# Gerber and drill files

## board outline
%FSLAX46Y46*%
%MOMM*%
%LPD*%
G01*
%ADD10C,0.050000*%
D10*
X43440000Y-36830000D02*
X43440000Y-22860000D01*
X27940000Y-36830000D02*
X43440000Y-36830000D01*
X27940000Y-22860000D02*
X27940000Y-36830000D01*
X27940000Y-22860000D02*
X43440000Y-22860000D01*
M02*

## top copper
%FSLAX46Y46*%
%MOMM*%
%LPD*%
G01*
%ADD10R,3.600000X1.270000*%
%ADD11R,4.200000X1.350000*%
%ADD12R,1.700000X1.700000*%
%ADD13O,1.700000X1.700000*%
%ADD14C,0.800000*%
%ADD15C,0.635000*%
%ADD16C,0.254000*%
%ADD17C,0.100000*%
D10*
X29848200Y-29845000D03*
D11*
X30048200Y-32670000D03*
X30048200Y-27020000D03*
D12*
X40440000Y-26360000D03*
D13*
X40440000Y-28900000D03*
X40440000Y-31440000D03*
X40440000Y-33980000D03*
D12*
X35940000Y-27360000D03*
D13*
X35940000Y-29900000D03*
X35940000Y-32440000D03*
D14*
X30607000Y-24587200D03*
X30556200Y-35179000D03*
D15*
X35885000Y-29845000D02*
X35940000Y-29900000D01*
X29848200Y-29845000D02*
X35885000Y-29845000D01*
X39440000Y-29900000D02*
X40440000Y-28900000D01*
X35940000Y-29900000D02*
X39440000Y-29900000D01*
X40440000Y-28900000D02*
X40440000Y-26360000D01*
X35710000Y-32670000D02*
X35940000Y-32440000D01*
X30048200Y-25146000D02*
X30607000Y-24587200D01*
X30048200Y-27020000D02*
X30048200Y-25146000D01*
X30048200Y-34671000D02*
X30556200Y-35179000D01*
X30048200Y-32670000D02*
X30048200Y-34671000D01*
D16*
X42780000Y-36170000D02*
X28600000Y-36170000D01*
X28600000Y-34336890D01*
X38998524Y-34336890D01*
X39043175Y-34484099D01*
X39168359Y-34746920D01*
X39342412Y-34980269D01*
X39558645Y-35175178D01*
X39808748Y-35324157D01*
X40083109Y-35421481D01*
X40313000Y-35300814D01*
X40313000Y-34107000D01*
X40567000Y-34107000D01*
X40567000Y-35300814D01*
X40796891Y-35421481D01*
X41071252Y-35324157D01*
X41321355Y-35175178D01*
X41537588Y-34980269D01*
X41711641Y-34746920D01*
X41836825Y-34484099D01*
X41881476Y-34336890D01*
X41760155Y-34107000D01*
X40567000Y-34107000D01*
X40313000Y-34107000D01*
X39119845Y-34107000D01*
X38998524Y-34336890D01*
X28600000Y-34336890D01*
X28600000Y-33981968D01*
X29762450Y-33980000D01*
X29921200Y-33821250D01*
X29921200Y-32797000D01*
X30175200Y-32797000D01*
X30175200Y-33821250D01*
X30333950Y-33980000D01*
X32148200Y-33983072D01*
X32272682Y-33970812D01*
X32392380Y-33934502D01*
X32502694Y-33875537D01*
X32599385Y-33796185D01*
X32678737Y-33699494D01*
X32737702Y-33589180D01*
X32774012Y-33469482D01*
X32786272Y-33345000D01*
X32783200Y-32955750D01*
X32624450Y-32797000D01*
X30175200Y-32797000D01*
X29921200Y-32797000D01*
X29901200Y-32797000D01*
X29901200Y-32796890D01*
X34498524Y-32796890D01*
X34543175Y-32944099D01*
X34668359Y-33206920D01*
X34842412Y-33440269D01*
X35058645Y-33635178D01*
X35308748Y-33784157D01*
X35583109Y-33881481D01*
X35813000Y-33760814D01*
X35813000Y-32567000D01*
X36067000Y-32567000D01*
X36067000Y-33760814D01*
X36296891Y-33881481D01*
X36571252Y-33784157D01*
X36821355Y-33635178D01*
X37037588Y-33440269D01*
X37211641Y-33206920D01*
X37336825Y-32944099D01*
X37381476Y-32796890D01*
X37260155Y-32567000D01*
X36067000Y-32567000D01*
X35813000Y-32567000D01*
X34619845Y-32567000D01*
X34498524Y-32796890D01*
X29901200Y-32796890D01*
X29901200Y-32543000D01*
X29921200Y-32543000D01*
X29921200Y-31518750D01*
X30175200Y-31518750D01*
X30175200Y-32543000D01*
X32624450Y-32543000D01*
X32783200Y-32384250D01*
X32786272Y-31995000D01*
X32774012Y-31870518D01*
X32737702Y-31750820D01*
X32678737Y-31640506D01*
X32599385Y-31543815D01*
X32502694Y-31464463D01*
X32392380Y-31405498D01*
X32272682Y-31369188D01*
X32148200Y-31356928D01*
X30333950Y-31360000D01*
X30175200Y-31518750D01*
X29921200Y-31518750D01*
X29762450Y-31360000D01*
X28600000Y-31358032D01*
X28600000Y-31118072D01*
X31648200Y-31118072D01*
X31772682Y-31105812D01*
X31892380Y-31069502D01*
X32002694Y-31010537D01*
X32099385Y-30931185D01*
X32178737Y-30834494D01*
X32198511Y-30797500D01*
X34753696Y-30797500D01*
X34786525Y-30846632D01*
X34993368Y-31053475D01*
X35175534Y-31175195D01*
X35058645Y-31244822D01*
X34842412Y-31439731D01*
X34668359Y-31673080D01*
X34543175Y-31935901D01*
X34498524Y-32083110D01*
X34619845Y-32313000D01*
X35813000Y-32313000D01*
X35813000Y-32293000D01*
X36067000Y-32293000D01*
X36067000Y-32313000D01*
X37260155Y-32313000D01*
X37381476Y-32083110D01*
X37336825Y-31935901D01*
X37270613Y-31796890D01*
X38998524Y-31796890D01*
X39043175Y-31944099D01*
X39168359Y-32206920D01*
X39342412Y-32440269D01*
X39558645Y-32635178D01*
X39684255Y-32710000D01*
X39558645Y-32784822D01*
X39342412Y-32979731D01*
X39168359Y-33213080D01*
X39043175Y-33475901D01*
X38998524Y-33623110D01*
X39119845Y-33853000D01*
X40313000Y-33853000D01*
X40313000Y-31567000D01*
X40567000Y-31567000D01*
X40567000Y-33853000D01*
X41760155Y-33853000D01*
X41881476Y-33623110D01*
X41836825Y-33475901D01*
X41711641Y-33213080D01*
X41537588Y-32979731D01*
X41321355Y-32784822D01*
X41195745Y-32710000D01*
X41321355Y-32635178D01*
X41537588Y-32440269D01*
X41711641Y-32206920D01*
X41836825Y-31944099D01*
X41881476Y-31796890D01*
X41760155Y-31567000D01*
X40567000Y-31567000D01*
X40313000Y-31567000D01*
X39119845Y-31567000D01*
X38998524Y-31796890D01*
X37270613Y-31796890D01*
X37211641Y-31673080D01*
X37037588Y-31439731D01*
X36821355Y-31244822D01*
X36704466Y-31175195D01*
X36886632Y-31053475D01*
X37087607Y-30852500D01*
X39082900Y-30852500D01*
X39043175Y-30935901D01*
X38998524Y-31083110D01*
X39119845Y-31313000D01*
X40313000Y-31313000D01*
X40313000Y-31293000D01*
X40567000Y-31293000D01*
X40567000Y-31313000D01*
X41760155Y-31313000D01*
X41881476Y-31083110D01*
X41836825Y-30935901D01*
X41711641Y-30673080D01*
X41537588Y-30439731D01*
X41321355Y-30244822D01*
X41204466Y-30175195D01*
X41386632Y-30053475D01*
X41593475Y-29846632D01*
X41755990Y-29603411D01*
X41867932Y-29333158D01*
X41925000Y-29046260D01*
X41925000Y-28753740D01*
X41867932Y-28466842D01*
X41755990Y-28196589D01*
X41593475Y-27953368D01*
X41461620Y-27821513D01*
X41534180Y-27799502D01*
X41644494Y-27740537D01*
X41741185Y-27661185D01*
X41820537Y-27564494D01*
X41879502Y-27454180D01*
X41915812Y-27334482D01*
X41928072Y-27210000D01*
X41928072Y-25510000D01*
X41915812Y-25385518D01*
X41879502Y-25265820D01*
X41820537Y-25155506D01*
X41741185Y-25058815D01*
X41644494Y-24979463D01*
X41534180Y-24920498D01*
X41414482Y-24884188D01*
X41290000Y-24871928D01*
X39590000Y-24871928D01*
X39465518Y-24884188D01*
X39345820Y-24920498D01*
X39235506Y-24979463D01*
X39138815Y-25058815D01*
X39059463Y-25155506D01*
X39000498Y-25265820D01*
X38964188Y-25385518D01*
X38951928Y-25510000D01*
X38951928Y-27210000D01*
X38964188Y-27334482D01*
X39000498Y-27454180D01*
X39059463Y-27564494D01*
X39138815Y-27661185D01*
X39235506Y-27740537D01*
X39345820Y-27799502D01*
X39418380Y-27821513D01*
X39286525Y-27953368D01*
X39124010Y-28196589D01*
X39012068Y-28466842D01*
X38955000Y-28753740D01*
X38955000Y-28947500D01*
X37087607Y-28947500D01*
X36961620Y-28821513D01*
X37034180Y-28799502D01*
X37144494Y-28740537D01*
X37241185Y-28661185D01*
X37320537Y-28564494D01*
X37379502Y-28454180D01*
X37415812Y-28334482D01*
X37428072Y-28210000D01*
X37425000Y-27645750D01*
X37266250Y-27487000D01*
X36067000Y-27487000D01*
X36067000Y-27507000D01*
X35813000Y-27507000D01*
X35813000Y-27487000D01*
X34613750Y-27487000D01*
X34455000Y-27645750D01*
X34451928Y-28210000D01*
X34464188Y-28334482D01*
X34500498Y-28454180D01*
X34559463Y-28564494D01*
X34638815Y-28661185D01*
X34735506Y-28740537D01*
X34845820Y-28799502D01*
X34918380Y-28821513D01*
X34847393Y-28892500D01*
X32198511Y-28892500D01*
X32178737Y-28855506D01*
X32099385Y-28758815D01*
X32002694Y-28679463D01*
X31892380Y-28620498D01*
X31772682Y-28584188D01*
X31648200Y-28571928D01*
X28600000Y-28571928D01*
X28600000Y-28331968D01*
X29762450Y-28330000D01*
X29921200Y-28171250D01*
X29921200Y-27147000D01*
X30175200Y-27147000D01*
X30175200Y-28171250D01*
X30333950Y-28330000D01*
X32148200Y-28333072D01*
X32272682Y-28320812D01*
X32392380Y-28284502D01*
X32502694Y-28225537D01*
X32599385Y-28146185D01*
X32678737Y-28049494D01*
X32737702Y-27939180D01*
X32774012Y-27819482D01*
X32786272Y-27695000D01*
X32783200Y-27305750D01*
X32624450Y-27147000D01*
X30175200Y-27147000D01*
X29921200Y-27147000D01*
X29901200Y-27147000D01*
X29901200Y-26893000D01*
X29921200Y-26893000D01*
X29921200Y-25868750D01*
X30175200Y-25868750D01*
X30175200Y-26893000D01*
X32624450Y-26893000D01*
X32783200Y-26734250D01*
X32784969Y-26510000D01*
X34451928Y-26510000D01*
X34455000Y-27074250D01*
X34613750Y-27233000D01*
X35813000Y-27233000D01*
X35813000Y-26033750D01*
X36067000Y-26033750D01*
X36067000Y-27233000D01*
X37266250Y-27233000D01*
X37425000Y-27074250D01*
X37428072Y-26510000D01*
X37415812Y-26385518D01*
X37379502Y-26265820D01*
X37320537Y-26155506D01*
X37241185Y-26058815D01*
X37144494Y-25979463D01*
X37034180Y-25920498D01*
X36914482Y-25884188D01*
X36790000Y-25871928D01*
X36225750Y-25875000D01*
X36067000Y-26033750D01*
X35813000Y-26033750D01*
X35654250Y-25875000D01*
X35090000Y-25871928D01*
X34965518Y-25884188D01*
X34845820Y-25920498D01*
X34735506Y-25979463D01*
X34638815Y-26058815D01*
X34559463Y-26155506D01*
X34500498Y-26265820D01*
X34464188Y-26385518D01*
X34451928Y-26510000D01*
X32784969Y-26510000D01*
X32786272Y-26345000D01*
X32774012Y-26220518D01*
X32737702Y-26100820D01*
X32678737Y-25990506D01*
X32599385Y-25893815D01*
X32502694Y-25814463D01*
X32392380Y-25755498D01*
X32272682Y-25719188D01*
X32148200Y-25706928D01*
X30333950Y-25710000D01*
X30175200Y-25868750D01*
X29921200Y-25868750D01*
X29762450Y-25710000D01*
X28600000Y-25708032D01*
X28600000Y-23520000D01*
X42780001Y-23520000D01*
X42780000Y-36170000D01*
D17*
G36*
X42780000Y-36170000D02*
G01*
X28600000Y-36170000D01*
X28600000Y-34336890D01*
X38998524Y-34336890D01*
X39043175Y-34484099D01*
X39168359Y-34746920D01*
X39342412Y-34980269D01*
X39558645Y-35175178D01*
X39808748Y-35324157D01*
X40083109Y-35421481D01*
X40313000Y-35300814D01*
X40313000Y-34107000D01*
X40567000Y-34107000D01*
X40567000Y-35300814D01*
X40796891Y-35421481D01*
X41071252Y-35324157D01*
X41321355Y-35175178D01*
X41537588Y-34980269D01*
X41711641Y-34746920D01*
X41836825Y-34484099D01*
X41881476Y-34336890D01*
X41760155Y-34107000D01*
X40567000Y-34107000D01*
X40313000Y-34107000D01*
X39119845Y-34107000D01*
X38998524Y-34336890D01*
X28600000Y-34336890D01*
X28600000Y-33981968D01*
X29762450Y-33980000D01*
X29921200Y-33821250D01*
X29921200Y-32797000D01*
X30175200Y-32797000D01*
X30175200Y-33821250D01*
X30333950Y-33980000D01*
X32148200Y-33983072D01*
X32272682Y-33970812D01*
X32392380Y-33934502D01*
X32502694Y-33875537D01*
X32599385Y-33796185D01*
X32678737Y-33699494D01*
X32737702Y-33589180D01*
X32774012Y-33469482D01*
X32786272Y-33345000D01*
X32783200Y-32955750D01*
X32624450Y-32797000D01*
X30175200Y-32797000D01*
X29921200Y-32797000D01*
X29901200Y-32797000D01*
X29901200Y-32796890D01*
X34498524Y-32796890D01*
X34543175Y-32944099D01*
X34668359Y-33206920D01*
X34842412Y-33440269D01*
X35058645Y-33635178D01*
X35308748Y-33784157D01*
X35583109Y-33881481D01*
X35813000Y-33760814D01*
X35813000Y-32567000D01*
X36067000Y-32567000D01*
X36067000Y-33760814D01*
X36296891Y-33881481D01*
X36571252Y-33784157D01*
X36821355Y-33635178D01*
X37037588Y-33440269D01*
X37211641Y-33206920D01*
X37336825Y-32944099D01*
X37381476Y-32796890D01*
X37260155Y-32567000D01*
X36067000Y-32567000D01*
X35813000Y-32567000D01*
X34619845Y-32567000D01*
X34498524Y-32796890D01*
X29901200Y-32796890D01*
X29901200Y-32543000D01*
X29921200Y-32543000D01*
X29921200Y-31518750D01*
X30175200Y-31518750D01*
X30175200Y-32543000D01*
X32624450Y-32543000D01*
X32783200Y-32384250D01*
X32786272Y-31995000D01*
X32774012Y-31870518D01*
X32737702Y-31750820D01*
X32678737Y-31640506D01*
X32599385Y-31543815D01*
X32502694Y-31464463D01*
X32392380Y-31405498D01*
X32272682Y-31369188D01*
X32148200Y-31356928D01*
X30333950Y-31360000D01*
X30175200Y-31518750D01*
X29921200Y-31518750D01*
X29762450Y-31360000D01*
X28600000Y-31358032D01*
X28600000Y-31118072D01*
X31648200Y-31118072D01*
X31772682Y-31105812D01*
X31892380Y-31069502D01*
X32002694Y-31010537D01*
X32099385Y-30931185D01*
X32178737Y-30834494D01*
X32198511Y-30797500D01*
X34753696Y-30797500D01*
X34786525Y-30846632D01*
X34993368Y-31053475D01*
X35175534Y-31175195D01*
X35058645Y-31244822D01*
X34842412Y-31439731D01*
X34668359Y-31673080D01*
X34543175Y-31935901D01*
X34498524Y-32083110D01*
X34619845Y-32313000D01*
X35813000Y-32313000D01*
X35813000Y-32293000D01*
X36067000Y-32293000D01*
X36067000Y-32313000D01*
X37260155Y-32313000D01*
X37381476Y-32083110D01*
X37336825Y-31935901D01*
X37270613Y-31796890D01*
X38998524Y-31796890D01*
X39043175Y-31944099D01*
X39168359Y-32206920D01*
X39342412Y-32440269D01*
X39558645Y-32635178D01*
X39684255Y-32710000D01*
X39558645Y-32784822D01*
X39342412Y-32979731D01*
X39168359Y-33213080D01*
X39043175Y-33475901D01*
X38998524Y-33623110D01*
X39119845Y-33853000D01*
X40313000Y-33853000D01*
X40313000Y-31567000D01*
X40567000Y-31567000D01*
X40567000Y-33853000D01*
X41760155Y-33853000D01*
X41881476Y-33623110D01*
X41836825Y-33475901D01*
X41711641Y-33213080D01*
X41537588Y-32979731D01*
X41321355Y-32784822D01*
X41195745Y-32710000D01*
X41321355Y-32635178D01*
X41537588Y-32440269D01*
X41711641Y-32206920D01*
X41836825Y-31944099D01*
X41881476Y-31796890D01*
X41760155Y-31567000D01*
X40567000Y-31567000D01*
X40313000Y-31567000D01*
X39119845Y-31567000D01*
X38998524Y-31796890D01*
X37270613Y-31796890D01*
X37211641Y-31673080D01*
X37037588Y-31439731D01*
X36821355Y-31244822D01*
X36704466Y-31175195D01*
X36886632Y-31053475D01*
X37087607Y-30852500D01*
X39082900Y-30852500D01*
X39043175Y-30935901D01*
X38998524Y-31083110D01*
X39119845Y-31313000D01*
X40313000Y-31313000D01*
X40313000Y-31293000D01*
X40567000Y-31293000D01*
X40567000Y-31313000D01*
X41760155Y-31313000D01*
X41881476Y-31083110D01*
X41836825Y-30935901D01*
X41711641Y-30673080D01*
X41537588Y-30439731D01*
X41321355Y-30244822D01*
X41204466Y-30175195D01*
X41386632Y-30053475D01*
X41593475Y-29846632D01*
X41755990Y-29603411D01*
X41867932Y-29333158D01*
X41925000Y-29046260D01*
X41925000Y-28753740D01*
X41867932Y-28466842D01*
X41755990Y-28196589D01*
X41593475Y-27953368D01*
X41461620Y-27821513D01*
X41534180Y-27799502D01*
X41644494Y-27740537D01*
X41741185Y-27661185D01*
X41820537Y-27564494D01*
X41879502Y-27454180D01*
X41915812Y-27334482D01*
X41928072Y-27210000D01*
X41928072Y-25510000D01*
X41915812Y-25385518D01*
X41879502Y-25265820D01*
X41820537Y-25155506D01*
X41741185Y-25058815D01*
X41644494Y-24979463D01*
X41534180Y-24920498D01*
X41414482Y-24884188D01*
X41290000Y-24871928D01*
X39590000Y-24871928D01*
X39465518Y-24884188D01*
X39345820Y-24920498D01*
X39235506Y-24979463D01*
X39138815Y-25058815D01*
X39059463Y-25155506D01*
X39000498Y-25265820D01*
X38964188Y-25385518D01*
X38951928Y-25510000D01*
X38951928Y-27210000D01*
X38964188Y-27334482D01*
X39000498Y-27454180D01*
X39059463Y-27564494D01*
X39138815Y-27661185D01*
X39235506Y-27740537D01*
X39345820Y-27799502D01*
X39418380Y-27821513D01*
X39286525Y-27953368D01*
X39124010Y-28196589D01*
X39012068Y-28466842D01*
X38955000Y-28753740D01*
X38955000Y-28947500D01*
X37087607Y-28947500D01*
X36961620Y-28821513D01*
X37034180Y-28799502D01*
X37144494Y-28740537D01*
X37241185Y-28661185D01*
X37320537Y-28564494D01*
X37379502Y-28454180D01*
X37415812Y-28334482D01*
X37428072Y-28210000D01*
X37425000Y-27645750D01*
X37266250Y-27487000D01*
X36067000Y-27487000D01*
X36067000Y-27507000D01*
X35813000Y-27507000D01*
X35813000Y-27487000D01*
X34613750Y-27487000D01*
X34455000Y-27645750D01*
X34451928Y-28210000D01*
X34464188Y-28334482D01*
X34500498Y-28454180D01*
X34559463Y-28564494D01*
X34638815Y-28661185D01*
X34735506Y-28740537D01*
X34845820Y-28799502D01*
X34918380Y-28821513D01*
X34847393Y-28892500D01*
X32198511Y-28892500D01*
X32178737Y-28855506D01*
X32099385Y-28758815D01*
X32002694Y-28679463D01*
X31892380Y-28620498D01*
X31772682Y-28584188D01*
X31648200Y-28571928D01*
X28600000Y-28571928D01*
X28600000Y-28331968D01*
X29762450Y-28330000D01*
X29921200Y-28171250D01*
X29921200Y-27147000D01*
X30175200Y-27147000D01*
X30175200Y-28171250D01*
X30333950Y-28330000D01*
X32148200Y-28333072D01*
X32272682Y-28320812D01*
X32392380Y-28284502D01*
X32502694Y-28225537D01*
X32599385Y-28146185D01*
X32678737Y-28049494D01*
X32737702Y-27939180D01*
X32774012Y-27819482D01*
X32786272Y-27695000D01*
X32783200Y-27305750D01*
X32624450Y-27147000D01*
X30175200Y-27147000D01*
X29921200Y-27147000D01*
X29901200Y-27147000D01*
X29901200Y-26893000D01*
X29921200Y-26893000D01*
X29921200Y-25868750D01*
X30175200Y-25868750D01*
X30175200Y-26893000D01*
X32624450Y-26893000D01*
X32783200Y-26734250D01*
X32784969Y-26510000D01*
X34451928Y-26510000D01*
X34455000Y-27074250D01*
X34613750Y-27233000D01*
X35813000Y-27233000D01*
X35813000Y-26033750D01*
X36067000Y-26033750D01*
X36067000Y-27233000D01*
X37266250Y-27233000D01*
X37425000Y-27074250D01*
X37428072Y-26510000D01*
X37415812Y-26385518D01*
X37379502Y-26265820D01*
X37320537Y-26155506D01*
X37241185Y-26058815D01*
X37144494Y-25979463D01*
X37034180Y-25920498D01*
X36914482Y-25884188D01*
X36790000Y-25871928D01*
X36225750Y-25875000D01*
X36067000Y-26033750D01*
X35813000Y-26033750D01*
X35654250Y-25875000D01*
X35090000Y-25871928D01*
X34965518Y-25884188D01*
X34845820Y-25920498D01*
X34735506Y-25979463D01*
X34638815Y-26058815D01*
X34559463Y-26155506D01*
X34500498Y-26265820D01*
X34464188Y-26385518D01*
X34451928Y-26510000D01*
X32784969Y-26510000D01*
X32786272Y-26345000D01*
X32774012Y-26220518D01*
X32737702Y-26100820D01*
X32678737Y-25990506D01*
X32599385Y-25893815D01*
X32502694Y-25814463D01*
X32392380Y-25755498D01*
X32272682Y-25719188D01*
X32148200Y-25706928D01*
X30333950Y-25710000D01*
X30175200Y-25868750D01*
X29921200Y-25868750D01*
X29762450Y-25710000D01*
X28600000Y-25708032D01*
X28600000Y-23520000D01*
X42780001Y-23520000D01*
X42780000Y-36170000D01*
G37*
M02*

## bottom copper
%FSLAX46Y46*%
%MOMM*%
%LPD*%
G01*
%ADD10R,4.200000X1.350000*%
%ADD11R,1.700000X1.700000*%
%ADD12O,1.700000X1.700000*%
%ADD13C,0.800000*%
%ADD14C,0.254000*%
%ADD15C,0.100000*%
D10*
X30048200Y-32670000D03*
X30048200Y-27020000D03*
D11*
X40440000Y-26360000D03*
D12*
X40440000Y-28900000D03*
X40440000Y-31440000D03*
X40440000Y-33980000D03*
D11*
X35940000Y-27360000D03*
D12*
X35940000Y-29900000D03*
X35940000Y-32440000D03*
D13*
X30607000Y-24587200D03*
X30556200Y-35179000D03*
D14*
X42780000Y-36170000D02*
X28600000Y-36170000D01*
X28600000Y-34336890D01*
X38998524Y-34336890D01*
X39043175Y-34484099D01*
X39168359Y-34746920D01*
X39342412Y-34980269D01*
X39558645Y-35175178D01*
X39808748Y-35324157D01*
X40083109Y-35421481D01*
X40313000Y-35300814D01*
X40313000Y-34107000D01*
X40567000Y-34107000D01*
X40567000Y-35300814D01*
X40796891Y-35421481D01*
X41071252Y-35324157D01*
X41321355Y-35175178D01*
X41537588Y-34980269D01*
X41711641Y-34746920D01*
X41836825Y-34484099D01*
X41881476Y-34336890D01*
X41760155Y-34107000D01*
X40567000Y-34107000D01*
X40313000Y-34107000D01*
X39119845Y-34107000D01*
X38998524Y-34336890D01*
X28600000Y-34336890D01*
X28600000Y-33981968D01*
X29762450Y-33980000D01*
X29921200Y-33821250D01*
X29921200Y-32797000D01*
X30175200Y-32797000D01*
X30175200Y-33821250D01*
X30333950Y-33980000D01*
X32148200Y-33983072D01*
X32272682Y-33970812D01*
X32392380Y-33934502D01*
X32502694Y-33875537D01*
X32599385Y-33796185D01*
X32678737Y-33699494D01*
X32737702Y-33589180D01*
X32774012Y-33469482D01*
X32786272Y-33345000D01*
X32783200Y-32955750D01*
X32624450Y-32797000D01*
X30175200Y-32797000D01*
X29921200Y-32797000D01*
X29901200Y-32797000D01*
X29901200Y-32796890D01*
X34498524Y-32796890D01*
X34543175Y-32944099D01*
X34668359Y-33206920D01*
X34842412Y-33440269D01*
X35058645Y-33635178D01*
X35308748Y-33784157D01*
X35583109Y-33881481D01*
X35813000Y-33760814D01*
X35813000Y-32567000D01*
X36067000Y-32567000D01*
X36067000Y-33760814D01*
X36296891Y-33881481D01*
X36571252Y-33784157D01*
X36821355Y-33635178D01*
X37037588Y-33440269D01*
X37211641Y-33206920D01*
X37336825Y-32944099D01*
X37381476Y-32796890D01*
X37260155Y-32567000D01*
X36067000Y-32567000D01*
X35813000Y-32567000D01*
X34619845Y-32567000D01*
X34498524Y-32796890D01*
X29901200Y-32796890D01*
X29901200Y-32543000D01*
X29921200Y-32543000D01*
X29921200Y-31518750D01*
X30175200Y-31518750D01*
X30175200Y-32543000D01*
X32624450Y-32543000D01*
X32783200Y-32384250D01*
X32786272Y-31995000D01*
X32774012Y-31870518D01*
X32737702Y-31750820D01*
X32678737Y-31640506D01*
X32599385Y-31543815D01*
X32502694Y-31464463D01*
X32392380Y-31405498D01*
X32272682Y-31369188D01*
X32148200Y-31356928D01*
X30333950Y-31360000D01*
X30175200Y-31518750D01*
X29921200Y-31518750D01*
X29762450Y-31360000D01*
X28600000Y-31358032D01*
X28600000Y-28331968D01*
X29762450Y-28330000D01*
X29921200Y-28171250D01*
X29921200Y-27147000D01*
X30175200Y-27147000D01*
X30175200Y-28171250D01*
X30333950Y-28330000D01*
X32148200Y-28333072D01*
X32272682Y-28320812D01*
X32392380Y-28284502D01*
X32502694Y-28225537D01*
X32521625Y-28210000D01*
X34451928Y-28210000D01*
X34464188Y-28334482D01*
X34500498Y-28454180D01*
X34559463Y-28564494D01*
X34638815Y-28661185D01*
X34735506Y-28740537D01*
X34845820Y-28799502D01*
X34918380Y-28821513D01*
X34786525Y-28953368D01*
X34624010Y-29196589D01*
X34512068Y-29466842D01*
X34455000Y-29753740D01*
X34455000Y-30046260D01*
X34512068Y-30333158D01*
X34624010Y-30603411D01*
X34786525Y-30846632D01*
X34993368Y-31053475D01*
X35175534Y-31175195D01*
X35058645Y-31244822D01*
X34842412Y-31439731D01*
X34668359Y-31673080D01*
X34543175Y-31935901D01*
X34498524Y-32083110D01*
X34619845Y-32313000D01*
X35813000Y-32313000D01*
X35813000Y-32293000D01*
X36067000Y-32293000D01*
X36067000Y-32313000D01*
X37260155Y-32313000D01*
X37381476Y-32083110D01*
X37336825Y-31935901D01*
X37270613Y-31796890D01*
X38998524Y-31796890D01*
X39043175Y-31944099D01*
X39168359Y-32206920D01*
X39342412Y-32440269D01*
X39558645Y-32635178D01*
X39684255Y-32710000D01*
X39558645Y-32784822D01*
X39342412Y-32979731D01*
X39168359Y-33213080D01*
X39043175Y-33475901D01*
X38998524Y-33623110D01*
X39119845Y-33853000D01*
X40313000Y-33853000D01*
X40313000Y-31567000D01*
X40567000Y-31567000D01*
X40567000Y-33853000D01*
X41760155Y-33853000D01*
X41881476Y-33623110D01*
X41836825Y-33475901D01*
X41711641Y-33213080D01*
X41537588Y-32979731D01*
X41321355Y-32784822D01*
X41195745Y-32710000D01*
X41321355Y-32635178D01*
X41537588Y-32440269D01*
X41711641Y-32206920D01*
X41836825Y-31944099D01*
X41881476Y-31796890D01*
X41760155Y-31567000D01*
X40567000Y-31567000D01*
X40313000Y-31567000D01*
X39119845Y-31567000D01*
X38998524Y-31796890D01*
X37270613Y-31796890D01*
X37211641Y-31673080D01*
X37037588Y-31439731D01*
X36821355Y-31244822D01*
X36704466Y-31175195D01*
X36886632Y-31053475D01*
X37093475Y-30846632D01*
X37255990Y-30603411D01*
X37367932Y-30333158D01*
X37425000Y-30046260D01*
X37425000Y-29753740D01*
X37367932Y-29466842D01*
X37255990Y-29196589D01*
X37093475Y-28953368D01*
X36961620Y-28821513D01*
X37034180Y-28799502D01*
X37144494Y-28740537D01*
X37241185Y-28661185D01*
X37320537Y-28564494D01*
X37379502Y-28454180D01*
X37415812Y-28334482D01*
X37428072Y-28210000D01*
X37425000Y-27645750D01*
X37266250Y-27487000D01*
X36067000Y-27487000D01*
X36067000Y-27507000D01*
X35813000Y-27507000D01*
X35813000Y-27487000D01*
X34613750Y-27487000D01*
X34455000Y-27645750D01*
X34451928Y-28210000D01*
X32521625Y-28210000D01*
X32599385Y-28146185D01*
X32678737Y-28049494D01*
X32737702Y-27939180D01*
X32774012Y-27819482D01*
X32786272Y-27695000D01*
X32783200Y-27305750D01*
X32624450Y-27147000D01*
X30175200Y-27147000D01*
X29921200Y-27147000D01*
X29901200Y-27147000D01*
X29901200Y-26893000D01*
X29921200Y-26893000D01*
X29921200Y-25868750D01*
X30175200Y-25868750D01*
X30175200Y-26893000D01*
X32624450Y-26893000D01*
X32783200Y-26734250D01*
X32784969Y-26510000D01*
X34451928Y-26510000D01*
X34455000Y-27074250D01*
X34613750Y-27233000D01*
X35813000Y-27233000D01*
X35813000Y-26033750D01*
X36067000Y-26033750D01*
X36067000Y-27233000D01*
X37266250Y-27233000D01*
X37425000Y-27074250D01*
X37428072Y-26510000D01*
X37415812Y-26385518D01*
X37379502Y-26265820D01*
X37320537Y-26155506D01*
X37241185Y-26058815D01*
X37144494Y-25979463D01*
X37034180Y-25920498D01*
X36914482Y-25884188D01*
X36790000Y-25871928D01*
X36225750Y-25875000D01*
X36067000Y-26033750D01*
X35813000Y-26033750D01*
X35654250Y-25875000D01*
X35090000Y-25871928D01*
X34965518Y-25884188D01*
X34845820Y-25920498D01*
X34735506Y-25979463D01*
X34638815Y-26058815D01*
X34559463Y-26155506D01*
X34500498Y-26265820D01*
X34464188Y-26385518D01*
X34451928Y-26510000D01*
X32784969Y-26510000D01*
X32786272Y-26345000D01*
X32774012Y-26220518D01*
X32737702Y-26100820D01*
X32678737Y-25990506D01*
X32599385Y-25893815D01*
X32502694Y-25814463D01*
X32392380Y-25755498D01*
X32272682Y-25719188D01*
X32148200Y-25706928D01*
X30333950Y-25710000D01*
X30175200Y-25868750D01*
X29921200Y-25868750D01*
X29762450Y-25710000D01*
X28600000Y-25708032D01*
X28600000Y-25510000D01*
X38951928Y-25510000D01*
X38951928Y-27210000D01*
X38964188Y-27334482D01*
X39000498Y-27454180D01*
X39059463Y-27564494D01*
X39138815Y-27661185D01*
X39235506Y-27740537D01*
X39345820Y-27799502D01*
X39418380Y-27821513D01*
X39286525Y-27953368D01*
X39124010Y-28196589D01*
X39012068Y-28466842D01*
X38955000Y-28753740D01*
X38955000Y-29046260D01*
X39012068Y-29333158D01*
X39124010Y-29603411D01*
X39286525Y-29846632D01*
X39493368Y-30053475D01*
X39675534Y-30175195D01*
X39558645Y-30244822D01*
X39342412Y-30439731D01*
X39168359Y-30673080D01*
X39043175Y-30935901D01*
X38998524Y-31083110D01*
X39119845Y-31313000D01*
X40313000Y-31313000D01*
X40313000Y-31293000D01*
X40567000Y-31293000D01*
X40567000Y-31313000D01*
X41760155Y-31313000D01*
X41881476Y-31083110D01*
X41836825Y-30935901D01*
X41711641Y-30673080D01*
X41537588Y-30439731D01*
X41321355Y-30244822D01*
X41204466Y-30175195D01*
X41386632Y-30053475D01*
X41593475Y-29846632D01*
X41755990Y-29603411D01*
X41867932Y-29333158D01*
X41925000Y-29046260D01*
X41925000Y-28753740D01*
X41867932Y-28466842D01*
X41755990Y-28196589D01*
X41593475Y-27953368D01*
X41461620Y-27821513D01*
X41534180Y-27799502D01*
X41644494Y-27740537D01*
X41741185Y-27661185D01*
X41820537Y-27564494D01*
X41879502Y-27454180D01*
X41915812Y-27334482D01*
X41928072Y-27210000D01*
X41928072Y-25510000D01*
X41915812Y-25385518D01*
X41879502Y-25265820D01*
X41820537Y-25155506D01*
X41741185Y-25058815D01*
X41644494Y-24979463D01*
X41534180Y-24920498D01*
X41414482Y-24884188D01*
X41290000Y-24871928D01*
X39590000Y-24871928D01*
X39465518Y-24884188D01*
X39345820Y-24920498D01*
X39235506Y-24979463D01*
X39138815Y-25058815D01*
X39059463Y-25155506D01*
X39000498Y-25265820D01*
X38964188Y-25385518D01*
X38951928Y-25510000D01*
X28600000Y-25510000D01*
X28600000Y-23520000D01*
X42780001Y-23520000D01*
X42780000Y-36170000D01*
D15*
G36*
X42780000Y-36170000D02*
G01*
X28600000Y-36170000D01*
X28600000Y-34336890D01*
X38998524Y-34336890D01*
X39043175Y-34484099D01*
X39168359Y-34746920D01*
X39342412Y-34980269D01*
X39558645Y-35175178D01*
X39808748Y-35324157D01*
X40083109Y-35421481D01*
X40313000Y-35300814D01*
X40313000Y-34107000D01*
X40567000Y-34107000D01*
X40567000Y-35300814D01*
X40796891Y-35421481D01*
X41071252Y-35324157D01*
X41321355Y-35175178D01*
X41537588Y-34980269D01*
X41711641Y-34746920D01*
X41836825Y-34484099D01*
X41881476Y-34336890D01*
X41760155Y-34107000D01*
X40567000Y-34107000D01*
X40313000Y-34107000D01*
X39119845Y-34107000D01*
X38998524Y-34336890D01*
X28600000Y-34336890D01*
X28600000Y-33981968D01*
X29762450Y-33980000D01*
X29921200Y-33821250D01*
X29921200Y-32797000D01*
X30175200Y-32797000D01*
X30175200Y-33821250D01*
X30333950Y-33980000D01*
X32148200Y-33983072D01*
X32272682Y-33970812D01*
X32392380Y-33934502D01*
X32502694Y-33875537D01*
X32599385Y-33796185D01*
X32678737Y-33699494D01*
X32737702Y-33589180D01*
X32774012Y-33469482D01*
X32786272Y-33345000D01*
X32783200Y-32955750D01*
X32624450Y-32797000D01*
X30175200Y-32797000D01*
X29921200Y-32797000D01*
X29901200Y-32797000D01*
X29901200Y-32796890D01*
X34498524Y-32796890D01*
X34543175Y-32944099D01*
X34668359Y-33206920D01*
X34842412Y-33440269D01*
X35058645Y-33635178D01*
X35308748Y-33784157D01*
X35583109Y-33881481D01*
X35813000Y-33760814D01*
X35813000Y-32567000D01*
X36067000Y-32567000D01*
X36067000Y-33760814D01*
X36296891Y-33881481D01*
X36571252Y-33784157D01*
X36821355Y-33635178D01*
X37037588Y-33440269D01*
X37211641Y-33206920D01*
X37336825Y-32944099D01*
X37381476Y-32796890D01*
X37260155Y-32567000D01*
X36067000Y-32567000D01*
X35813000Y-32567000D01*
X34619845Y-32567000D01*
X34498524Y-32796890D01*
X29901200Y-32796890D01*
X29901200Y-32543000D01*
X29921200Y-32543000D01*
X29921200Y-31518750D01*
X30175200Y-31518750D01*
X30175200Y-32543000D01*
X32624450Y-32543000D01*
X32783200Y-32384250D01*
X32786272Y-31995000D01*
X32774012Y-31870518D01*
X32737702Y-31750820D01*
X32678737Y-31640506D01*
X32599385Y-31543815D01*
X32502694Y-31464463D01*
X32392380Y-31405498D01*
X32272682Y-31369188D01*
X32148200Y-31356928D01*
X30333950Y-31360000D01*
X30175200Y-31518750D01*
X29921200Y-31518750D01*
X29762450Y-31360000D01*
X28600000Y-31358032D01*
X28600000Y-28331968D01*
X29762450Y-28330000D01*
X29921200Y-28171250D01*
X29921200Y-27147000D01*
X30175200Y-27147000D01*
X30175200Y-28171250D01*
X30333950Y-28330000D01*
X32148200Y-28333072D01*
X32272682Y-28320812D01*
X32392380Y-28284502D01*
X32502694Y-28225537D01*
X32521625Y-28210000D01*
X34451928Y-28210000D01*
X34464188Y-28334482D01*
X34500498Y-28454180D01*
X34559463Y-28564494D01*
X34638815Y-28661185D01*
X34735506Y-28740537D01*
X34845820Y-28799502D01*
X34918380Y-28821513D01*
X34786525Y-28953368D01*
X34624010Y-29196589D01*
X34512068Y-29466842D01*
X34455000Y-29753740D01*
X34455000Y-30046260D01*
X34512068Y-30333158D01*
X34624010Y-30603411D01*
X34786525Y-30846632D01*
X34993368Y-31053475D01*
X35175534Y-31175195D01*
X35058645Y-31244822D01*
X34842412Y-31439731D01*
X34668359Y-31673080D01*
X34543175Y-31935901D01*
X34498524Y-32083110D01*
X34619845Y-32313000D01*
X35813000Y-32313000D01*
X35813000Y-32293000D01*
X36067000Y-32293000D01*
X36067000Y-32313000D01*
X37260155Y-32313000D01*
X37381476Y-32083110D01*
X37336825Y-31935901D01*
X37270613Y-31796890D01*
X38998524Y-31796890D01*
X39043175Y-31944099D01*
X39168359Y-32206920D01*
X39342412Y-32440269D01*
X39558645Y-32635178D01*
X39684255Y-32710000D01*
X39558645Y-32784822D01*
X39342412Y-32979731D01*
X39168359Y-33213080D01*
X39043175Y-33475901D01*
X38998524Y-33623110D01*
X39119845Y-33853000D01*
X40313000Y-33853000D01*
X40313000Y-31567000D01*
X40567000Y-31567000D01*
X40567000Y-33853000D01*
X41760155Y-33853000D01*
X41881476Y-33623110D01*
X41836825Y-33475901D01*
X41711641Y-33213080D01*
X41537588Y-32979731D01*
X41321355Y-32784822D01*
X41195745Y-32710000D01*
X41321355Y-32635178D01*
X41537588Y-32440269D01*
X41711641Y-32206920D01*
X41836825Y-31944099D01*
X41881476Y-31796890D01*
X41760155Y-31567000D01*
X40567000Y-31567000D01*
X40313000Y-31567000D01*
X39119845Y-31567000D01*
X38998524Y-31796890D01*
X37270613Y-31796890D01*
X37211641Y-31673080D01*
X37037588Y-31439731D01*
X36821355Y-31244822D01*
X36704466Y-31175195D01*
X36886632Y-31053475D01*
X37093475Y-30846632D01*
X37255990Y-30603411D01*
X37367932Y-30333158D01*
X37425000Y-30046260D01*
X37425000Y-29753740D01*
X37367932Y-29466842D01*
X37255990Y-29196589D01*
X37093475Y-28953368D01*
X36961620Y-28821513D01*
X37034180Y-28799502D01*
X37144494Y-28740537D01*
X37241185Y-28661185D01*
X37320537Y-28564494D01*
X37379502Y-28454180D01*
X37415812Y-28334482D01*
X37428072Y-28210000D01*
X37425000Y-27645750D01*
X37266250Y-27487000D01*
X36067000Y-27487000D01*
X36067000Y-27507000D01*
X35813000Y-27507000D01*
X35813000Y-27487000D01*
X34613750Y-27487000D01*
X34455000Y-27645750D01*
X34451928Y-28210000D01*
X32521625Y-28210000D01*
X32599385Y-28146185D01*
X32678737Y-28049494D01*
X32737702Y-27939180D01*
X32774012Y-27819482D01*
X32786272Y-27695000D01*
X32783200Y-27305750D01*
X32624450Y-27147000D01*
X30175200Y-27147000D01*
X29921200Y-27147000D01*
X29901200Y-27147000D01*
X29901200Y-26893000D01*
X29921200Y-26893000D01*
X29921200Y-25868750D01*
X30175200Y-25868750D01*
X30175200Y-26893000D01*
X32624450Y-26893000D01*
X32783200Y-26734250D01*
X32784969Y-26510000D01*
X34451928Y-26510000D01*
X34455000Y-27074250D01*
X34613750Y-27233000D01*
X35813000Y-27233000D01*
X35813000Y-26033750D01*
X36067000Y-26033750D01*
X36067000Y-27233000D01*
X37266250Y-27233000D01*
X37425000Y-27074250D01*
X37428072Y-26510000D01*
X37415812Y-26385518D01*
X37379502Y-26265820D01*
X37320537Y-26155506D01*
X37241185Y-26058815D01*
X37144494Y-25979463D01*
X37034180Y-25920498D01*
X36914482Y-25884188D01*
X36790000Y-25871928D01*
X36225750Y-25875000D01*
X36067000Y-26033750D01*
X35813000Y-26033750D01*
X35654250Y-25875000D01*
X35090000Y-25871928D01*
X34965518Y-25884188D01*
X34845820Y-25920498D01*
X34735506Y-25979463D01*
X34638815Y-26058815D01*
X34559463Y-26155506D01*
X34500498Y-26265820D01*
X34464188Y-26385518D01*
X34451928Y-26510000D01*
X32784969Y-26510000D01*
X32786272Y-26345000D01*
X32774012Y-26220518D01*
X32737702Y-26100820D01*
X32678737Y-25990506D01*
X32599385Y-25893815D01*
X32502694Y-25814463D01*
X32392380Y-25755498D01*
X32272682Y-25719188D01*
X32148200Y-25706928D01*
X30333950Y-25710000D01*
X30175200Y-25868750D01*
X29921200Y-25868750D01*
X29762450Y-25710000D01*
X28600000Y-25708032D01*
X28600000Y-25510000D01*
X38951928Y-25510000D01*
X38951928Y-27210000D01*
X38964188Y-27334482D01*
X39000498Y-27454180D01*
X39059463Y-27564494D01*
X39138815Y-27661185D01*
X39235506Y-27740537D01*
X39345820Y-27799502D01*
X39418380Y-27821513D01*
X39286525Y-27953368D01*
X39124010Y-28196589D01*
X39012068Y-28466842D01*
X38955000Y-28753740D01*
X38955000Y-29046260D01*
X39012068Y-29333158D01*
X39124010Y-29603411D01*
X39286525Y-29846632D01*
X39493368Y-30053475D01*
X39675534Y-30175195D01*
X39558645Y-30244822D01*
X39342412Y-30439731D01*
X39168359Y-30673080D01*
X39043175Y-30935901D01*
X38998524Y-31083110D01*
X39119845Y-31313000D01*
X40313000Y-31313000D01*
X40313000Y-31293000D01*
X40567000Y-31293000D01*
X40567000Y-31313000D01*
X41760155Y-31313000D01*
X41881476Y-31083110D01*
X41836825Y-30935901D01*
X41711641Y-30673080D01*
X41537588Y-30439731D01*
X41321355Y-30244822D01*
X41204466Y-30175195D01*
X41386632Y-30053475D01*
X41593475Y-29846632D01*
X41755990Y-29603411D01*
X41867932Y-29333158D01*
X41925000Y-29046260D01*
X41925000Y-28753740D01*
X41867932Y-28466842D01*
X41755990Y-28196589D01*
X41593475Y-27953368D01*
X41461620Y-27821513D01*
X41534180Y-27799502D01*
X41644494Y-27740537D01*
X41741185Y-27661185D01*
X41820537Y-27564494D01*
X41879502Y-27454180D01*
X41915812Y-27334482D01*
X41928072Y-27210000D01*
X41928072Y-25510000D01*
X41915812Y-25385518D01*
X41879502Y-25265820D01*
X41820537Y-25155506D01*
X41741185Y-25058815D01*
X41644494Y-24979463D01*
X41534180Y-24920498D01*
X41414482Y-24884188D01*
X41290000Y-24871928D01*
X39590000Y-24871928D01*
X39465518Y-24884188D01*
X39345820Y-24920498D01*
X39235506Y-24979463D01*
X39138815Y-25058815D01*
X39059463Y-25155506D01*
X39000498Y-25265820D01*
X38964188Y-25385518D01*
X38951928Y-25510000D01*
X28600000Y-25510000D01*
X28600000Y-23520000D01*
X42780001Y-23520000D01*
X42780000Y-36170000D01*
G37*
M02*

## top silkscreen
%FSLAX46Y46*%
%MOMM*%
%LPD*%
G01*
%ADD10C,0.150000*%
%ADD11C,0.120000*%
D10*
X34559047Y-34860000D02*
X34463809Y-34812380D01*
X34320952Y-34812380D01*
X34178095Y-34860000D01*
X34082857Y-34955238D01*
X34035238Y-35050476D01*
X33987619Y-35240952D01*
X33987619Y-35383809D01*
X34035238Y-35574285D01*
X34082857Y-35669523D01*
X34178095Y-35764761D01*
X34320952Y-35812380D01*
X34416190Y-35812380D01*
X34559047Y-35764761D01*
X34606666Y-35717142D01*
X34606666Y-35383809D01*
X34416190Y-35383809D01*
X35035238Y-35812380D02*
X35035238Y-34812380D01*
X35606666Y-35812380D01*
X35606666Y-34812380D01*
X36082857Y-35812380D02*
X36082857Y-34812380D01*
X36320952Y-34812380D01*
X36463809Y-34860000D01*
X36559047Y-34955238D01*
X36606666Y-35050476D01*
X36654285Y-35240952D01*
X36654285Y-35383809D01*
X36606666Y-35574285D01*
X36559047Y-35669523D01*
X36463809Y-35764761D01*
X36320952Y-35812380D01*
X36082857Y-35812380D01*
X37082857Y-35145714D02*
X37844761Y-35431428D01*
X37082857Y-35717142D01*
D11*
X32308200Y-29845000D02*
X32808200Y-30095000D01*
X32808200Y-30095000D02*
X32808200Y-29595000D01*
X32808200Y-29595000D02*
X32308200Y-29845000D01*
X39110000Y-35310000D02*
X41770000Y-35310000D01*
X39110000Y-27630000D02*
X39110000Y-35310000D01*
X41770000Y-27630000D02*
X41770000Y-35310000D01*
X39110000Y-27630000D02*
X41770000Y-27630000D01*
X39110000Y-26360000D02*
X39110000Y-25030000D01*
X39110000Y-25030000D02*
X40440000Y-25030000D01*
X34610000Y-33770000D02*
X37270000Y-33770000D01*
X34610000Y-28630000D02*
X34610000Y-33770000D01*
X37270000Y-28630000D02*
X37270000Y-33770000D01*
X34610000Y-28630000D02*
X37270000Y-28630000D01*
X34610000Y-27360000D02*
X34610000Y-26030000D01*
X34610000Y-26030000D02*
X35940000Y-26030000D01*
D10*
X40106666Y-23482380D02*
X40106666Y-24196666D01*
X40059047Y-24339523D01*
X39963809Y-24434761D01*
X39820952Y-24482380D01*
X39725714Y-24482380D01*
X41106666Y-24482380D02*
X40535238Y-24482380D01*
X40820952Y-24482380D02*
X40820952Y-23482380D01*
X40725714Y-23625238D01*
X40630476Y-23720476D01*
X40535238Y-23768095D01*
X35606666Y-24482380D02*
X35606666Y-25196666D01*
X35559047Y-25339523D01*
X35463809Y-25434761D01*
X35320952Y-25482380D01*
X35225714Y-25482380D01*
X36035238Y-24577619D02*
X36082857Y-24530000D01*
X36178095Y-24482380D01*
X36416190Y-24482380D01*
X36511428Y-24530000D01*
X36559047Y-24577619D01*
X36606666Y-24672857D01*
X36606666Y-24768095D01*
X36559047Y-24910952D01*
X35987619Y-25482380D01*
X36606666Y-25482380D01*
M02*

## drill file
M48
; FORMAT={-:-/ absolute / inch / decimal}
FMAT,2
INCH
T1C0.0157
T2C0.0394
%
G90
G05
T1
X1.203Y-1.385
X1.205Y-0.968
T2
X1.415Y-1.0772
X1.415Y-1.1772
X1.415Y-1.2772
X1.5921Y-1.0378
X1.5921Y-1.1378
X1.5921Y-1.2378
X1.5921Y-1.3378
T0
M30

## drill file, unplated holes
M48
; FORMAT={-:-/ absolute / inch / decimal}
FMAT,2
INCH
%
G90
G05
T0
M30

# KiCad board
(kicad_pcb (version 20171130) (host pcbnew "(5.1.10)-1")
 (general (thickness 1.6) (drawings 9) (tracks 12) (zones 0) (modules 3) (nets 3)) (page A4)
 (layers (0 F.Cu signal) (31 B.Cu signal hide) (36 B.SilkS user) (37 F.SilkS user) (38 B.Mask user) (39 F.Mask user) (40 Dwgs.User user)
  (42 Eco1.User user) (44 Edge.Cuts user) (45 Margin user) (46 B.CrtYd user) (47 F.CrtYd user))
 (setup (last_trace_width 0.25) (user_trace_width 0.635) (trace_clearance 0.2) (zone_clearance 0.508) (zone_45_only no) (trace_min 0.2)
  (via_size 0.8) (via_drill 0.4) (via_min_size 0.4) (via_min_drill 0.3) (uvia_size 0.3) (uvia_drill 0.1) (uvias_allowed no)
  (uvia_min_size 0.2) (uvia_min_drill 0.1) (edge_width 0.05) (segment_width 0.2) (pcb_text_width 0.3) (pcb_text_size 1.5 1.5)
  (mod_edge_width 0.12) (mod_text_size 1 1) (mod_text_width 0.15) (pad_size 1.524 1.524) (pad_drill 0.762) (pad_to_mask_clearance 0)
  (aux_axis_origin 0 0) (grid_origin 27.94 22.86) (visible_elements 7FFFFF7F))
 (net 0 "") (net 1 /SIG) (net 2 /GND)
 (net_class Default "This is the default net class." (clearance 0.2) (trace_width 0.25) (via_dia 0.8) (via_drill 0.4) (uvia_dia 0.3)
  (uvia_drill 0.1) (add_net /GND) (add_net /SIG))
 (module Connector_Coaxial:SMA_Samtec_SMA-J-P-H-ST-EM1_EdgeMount (layer F.Cu) (at 30.0482 29.845 180)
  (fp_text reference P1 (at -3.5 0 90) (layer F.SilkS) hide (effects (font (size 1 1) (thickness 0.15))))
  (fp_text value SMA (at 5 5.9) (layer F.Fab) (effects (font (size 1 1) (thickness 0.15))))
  (fp_line (start -2.26 0) (end -2.76 -0.25) (layer F.SilkS) (width 0.12))
  (fp_line (start -2.76 -0.25) (end -2.76 0.25) (layer F.SilkS) (width 0.12))
  (fp_line (start -2.76 0.25) (end -2.26 0) (layer F.SilkS) (width 0.12))
  (pad 1 smd rect (at 0.2 0 270) (size 1.27 3.6) (layers F.Cu F.Paste F.Mask) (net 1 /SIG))
  (pad 2 smd rect (at 0 -2.825 270) (size 1.35 4.2) (layers F.Cu F.Paste F.Mask) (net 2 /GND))
  (pad 2 smd rect (at 0 2.825 270) (size 1.35 4.2) (layers F.Cu F.Paste F.Mask) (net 2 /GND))
  (pad 2 smd rect (at 0 -2.825 270) (size 1.35 4.2) (layers B.Cu B.Paste B.Mask) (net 2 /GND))
  (pad 2 smd rect (at 0 2.825 270) (size 1.35 4.2) (layers B.Cu B.Paste B.Mask) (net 2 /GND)))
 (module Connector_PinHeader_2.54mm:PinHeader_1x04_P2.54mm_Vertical (layer F.Cu) (at 40.44 26.36)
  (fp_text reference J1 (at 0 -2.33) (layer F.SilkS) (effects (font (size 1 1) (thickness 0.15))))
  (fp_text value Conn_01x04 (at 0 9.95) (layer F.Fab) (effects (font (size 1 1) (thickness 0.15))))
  (fp_line (start -1.33 8.95) (end 1.33 8.95) (layer F.SilkS) (width 0.12))
  (fp_line (start -1.33 1.27) (end -1.33 8.95) (layer F.SilkS) (width 0.12))
  (fp_line (start 1.33 1.27) (end 1.33 8.95) (layer F.SilkS) (width 0.12))
  (fp_line (start -1.33 1.27) (end 1.33 1.27) (layer F.SilkS) (width 0.12))
  (fp_line (start -1.33 0) (end -1.33 -1.33) (layer F.SilkS) (width 0.12))
  (fp_line (start -1.33 -1.33) (end 0 -1.33) (layer F.SilkS) (width 0.12))
  (pad 1 thru_hole rect (at 0 0) (size 1.7 1.7) (drill 1) (layers *.Cu *.Mask) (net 1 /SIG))
  (pad 2 thru_hole oval (at 0 2.54) (size 1.7 1.7) (drill 1) (layers *.Cu *.Mask) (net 1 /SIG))
  (pad 3 thru_hole oval (at 0 5.08) (size 1.7 1.7) (drill 1) (layers *.Cu *.Mask) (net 2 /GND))
  (pad 4 thru_hole oval (at 0 7.62) (size 1.7 1.7) (drill 1) (layers *.Cu *.Mask) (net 2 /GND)))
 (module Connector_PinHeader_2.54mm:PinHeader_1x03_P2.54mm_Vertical (layer F.Cu) (at 35.94 27.36)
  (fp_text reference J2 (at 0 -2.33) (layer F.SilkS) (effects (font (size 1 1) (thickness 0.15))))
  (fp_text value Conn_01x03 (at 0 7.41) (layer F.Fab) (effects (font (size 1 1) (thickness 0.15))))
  (fp_line (start -1.33 6.41) (end 1.33 6.41) (layer F.SilkS) (width 0.12))
  (fp_line (start -1.33 1.27) (end -1.33 6.41) (layer F.SilkS) (width 0.12))
  (fp_line (start 1.33 1.27) (end 1.33 6.41) (layer F.SilkS) (width 0.12))
  (fp_line (start -1.33 1.27) (end 1.33 1.27) (layer F.SilkS) (width 0.12))
  (fp_line (start -1.33 0) (end -1.33 -1.33) (layer F.SilkS) (width 0.12))
  (fp_line (start -1.33 -1.33) (end 0 -1.33) (layer F.SilkS) (width 0.12))
  (pad 1 thru_hole rect (at 0 0) (size 1.7 1.7) (drill 1) (layers *.Cu *.Mask) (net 2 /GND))
  (pad 2 thru_hole oval (at 0 2.54) (size 1.7 1.7) (drill 1) (layers *.Cu *.Mask) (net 1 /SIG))
  (pad 3 thru_hole oval (at 0 5.08) (size 1.7 1.7) (drill 1) (layers *.Cu *.Mask) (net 2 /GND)))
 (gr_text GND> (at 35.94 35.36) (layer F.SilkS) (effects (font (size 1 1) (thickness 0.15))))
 (gr_line (start 43.44 36.83) (end 43.44 22.86) (layer Edge.Cuts) (width 0.05))
 (gr_line (start 27.94 36.83) (end 43.44 36.83) (layer Edge.Cuts) (width 0.05))
 (gr_line (start 27.94 22.86) (end 27.94 36.83) (layer Edge.Cuts) (width 0.05))
 (gr_line (start 27.94 22.86) (end 43.44 22.86) (layer Edge.Cuts) (width 0.05))
 (segment (start 35.885 29.845) (end 35.94 29.9) (width 0.635) (layer F.Cu) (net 1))
 (segment (start 29.8482 29.845) (end 35.885 29.845) (width 0.635) (layer F.Cu) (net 1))
 (segment (start 39.44 29.9) (end 40.44 28.9) (width 0.635) (layer F.Cu) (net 1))
 (segment (start 35.94 29.9) (end 39.44 29.9) (width 0.635) (layer F.Cu) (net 1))
 (segment (start 40.44 28.9) (end 40.44 26.36) (width 0.635) (layer F.Cu) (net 1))
 (via (at 30.607 24.5872) (size 0.8) (drill 0.4) (layers F.Cu B.Cu) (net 2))
 (via (at 30.5562 35.179) (size 0.8) (drill 0.4) (layers F.Cu B.Cu) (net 2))
 (segment (start 35.71 32.67) (end 35.94 32.44) (width 0.635) (layer F.Cu) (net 2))
 (segment (start 30.0482 25.146) (end 30.607 24.5872) (width 0.635) (layer F.Cu) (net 2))
 (segment (start 30.0482 27.02) (end 30.0482 25.146) (width 0.635) (layer F.Cu) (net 2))
 (segment (start 30.0482 34.671) (end 30.5562 35.179) (width 0.635) (layer F.Cu) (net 2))
 (segment (start 30.0482 32.67) (end 30.0482 34.671) (width 0.635) (layer F.Cu) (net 2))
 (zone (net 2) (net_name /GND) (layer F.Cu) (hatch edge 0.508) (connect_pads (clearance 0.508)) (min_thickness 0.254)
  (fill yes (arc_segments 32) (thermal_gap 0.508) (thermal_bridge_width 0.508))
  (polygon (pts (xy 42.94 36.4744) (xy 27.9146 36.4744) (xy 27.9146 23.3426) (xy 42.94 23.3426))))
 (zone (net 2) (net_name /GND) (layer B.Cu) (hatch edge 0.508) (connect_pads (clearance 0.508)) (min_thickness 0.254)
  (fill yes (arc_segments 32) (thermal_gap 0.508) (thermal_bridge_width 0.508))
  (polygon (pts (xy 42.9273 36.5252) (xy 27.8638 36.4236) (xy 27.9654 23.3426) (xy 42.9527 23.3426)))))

